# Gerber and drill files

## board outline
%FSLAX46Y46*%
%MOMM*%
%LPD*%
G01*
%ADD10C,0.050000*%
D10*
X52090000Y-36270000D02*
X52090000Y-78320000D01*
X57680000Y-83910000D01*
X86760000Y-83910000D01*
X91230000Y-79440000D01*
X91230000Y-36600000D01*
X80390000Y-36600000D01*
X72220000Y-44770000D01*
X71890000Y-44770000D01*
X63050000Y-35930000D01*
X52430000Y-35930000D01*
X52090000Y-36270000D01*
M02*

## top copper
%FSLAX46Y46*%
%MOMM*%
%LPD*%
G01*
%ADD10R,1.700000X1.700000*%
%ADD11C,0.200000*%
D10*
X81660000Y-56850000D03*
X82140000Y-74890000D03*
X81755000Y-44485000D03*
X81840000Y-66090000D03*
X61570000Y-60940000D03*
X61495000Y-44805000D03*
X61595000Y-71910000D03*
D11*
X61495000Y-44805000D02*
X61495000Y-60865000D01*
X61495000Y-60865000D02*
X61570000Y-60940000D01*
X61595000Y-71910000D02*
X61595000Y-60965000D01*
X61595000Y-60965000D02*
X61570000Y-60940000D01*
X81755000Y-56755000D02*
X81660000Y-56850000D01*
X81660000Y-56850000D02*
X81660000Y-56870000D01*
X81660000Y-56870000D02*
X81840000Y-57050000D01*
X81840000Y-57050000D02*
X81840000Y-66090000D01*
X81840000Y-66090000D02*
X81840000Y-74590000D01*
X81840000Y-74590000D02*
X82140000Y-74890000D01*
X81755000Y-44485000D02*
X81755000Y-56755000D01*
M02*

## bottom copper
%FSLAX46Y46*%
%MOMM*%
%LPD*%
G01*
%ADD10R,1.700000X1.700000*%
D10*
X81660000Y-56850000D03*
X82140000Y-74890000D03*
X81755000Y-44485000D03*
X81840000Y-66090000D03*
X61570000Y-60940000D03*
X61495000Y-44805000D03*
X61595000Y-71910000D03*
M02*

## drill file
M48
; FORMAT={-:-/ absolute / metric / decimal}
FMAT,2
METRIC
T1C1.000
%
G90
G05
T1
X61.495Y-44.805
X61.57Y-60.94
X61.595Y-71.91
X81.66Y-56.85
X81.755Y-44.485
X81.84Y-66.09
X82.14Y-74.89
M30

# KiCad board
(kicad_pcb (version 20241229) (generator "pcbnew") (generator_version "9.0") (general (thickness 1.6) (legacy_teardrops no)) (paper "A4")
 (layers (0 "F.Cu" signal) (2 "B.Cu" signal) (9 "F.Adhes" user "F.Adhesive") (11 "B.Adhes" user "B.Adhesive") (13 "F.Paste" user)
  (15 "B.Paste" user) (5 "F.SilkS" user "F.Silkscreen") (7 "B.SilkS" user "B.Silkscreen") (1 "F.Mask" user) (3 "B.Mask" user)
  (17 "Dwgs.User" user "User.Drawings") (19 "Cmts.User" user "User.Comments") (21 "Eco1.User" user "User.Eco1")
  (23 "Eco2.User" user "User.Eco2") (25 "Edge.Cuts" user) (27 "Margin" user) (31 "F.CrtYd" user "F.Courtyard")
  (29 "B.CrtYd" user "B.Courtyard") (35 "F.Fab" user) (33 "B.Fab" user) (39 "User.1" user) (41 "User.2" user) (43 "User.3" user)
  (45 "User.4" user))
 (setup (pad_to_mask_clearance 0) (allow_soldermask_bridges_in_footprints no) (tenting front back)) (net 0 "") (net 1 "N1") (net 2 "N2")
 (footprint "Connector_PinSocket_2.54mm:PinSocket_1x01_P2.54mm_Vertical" (layer "F.Cu") (at 81.66 56.85)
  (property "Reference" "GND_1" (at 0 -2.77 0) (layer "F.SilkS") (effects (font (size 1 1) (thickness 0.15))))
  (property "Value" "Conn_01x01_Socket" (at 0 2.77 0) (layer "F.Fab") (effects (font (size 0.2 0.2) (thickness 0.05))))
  (pad "1" thru_hole rect (at 0 0) (size 1.7 1.7) (drill 1) (layers "*.Cu" "*.Mask") (remove_unused_layers no) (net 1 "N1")))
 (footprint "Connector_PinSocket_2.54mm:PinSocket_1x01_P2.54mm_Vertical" (layer "F.Cu") (at 82.14 74.89)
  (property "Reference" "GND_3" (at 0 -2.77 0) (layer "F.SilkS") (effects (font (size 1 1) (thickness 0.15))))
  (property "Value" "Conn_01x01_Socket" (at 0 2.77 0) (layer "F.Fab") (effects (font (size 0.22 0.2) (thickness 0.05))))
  (pad "1" thru_hole rect (at 0 0) (size 1.7 1.7) (drill 1) (layers "*.Cu" "*.Mask") (remove_unused_layers no) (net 1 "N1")))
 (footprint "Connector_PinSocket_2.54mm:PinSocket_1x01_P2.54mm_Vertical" (layer "F.Cu") (at 81.755 44.485)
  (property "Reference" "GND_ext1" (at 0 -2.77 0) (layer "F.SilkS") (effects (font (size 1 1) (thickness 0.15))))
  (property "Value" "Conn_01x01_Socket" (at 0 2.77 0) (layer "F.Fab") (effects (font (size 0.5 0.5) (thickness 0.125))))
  (pad "1" thru_hole rect (at 0 0) (size 1.7 1.7) (drill 1) (layers "*.Cu" "*.Mask") (remove_unused_layers no) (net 1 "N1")))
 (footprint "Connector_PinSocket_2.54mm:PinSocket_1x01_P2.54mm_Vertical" (layer "F.Cu") (at 81.84 66.09)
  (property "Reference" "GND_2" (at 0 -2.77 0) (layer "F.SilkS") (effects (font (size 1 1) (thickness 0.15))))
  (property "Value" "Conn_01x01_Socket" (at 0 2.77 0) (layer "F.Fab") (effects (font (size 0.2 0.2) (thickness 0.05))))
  (pad "1" thru_hole rect (at 0 0) (size 1.7 1.7) (drill 1) (layers "*.Cu" "*.Mask") (remove_unused_layers no) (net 1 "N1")))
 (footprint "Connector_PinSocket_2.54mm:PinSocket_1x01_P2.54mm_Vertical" (layer "F.Cu") (at 61.57 60.94)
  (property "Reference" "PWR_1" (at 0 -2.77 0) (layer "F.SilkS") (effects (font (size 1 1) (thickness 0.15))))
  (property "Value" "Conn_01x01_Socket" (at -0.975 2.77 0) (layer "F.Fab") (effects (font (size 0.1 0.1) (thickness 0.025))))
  (pad "1" thru_hole rect (at 0 0) (size 1.7 1.7) (drill 1) (layers "*.Cu" "*.Mask") (remove_unused_layers no) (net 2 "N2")))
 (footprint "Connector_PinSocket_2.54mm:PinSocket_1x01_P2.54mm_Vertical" (layer "F.Cu") (at 61.495 44.805)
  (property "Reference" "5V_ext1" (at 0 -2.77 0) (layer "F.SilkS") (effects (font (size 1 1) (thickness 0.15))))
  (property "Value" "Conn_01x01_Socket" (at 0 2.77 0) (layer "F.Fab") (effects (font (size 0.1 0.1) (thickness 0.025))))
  (pad "1" thru_hole rect (at 0 0) (size 1.7 1.7) (drill 1) (layers "*.Cu" "*.Mask") (remove_unused_layers no) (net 2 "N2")))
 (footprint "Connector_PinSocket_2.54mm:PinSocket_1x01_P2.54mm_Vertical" (layer "F.Cu") (at 61.595 71.91)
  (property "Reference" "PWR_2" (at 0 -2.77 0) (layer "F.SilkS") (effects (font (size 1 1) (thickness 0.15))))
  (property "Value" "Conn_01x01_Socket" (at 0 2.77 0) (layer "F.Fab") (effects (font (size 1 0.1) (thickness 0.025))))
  (pad "1" thru_hole rect (at 0 0) (size 1.7 1.7) (drill 1) (layers "*.Cu" "*.Mask") (remove_unused_layers no) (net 2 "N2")))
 (gr_poly
  (pts (xy 52.09 36.27) (xy 52.09 78.32) (xy 57.68 83.91) (xy 86.76 83.91) (xy 91.23 79.44) (xy 91.23 36.6) (xy 80.39 36.6) (xy 72.22 44.77)
   (xy 71.89 44.77) (xy 63.05 35.93) (xy 52.43 35.93))
  (stroke (width 0.05) (type solid)) (fill no) (layer "Edge.Cuts"))
 (segment (start 61.495 44.805) (end 61.495 60.865) (width 0.2) (layer "F.Cu") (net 2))
 (segment (start 61.495 60.865) (end 61.57 60.94) (width 0.2) (layer "F.Cu") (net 2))
 (segment (start 61.595 71.91) (end 61.595 60.965) (width 0.2) (layer "F.Cu") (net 2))
 (segment (start 61.595 60.965) (end 61.57 60.94) (width 0.2) (layer "F.Cu") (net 2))
 (segment (start 81.755 56.755) (end 81.66 56.85) (width 0.2) (layer "F.Cu") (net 1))
 (segment (start 81.66 56.85) (end 81.66 56.87) (width 0.2) (layer "F.Cu") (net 1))
 (segment (start 81.66 56.87) (end 81.84 57.05) (width 0.2) (layer "F.Cu") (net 1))
 (segment (start 81.84 57.05) (end 81.84 66.09) (width 0.2) (layer "F.Cu") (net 1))
 (segment (start 81.84 66.09) (end 81.84 74.59) (width 0.2) (layer "F.Cu") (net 1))
 (segment (start 81.84 74.59) (end 82.14 74.89) (width 0.2) (layer "F.Cu") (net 1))
 (segment (start 81.755 44.485) (end 81.755 56.755) (width 0.2) (layer "F.Cu") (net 1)))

